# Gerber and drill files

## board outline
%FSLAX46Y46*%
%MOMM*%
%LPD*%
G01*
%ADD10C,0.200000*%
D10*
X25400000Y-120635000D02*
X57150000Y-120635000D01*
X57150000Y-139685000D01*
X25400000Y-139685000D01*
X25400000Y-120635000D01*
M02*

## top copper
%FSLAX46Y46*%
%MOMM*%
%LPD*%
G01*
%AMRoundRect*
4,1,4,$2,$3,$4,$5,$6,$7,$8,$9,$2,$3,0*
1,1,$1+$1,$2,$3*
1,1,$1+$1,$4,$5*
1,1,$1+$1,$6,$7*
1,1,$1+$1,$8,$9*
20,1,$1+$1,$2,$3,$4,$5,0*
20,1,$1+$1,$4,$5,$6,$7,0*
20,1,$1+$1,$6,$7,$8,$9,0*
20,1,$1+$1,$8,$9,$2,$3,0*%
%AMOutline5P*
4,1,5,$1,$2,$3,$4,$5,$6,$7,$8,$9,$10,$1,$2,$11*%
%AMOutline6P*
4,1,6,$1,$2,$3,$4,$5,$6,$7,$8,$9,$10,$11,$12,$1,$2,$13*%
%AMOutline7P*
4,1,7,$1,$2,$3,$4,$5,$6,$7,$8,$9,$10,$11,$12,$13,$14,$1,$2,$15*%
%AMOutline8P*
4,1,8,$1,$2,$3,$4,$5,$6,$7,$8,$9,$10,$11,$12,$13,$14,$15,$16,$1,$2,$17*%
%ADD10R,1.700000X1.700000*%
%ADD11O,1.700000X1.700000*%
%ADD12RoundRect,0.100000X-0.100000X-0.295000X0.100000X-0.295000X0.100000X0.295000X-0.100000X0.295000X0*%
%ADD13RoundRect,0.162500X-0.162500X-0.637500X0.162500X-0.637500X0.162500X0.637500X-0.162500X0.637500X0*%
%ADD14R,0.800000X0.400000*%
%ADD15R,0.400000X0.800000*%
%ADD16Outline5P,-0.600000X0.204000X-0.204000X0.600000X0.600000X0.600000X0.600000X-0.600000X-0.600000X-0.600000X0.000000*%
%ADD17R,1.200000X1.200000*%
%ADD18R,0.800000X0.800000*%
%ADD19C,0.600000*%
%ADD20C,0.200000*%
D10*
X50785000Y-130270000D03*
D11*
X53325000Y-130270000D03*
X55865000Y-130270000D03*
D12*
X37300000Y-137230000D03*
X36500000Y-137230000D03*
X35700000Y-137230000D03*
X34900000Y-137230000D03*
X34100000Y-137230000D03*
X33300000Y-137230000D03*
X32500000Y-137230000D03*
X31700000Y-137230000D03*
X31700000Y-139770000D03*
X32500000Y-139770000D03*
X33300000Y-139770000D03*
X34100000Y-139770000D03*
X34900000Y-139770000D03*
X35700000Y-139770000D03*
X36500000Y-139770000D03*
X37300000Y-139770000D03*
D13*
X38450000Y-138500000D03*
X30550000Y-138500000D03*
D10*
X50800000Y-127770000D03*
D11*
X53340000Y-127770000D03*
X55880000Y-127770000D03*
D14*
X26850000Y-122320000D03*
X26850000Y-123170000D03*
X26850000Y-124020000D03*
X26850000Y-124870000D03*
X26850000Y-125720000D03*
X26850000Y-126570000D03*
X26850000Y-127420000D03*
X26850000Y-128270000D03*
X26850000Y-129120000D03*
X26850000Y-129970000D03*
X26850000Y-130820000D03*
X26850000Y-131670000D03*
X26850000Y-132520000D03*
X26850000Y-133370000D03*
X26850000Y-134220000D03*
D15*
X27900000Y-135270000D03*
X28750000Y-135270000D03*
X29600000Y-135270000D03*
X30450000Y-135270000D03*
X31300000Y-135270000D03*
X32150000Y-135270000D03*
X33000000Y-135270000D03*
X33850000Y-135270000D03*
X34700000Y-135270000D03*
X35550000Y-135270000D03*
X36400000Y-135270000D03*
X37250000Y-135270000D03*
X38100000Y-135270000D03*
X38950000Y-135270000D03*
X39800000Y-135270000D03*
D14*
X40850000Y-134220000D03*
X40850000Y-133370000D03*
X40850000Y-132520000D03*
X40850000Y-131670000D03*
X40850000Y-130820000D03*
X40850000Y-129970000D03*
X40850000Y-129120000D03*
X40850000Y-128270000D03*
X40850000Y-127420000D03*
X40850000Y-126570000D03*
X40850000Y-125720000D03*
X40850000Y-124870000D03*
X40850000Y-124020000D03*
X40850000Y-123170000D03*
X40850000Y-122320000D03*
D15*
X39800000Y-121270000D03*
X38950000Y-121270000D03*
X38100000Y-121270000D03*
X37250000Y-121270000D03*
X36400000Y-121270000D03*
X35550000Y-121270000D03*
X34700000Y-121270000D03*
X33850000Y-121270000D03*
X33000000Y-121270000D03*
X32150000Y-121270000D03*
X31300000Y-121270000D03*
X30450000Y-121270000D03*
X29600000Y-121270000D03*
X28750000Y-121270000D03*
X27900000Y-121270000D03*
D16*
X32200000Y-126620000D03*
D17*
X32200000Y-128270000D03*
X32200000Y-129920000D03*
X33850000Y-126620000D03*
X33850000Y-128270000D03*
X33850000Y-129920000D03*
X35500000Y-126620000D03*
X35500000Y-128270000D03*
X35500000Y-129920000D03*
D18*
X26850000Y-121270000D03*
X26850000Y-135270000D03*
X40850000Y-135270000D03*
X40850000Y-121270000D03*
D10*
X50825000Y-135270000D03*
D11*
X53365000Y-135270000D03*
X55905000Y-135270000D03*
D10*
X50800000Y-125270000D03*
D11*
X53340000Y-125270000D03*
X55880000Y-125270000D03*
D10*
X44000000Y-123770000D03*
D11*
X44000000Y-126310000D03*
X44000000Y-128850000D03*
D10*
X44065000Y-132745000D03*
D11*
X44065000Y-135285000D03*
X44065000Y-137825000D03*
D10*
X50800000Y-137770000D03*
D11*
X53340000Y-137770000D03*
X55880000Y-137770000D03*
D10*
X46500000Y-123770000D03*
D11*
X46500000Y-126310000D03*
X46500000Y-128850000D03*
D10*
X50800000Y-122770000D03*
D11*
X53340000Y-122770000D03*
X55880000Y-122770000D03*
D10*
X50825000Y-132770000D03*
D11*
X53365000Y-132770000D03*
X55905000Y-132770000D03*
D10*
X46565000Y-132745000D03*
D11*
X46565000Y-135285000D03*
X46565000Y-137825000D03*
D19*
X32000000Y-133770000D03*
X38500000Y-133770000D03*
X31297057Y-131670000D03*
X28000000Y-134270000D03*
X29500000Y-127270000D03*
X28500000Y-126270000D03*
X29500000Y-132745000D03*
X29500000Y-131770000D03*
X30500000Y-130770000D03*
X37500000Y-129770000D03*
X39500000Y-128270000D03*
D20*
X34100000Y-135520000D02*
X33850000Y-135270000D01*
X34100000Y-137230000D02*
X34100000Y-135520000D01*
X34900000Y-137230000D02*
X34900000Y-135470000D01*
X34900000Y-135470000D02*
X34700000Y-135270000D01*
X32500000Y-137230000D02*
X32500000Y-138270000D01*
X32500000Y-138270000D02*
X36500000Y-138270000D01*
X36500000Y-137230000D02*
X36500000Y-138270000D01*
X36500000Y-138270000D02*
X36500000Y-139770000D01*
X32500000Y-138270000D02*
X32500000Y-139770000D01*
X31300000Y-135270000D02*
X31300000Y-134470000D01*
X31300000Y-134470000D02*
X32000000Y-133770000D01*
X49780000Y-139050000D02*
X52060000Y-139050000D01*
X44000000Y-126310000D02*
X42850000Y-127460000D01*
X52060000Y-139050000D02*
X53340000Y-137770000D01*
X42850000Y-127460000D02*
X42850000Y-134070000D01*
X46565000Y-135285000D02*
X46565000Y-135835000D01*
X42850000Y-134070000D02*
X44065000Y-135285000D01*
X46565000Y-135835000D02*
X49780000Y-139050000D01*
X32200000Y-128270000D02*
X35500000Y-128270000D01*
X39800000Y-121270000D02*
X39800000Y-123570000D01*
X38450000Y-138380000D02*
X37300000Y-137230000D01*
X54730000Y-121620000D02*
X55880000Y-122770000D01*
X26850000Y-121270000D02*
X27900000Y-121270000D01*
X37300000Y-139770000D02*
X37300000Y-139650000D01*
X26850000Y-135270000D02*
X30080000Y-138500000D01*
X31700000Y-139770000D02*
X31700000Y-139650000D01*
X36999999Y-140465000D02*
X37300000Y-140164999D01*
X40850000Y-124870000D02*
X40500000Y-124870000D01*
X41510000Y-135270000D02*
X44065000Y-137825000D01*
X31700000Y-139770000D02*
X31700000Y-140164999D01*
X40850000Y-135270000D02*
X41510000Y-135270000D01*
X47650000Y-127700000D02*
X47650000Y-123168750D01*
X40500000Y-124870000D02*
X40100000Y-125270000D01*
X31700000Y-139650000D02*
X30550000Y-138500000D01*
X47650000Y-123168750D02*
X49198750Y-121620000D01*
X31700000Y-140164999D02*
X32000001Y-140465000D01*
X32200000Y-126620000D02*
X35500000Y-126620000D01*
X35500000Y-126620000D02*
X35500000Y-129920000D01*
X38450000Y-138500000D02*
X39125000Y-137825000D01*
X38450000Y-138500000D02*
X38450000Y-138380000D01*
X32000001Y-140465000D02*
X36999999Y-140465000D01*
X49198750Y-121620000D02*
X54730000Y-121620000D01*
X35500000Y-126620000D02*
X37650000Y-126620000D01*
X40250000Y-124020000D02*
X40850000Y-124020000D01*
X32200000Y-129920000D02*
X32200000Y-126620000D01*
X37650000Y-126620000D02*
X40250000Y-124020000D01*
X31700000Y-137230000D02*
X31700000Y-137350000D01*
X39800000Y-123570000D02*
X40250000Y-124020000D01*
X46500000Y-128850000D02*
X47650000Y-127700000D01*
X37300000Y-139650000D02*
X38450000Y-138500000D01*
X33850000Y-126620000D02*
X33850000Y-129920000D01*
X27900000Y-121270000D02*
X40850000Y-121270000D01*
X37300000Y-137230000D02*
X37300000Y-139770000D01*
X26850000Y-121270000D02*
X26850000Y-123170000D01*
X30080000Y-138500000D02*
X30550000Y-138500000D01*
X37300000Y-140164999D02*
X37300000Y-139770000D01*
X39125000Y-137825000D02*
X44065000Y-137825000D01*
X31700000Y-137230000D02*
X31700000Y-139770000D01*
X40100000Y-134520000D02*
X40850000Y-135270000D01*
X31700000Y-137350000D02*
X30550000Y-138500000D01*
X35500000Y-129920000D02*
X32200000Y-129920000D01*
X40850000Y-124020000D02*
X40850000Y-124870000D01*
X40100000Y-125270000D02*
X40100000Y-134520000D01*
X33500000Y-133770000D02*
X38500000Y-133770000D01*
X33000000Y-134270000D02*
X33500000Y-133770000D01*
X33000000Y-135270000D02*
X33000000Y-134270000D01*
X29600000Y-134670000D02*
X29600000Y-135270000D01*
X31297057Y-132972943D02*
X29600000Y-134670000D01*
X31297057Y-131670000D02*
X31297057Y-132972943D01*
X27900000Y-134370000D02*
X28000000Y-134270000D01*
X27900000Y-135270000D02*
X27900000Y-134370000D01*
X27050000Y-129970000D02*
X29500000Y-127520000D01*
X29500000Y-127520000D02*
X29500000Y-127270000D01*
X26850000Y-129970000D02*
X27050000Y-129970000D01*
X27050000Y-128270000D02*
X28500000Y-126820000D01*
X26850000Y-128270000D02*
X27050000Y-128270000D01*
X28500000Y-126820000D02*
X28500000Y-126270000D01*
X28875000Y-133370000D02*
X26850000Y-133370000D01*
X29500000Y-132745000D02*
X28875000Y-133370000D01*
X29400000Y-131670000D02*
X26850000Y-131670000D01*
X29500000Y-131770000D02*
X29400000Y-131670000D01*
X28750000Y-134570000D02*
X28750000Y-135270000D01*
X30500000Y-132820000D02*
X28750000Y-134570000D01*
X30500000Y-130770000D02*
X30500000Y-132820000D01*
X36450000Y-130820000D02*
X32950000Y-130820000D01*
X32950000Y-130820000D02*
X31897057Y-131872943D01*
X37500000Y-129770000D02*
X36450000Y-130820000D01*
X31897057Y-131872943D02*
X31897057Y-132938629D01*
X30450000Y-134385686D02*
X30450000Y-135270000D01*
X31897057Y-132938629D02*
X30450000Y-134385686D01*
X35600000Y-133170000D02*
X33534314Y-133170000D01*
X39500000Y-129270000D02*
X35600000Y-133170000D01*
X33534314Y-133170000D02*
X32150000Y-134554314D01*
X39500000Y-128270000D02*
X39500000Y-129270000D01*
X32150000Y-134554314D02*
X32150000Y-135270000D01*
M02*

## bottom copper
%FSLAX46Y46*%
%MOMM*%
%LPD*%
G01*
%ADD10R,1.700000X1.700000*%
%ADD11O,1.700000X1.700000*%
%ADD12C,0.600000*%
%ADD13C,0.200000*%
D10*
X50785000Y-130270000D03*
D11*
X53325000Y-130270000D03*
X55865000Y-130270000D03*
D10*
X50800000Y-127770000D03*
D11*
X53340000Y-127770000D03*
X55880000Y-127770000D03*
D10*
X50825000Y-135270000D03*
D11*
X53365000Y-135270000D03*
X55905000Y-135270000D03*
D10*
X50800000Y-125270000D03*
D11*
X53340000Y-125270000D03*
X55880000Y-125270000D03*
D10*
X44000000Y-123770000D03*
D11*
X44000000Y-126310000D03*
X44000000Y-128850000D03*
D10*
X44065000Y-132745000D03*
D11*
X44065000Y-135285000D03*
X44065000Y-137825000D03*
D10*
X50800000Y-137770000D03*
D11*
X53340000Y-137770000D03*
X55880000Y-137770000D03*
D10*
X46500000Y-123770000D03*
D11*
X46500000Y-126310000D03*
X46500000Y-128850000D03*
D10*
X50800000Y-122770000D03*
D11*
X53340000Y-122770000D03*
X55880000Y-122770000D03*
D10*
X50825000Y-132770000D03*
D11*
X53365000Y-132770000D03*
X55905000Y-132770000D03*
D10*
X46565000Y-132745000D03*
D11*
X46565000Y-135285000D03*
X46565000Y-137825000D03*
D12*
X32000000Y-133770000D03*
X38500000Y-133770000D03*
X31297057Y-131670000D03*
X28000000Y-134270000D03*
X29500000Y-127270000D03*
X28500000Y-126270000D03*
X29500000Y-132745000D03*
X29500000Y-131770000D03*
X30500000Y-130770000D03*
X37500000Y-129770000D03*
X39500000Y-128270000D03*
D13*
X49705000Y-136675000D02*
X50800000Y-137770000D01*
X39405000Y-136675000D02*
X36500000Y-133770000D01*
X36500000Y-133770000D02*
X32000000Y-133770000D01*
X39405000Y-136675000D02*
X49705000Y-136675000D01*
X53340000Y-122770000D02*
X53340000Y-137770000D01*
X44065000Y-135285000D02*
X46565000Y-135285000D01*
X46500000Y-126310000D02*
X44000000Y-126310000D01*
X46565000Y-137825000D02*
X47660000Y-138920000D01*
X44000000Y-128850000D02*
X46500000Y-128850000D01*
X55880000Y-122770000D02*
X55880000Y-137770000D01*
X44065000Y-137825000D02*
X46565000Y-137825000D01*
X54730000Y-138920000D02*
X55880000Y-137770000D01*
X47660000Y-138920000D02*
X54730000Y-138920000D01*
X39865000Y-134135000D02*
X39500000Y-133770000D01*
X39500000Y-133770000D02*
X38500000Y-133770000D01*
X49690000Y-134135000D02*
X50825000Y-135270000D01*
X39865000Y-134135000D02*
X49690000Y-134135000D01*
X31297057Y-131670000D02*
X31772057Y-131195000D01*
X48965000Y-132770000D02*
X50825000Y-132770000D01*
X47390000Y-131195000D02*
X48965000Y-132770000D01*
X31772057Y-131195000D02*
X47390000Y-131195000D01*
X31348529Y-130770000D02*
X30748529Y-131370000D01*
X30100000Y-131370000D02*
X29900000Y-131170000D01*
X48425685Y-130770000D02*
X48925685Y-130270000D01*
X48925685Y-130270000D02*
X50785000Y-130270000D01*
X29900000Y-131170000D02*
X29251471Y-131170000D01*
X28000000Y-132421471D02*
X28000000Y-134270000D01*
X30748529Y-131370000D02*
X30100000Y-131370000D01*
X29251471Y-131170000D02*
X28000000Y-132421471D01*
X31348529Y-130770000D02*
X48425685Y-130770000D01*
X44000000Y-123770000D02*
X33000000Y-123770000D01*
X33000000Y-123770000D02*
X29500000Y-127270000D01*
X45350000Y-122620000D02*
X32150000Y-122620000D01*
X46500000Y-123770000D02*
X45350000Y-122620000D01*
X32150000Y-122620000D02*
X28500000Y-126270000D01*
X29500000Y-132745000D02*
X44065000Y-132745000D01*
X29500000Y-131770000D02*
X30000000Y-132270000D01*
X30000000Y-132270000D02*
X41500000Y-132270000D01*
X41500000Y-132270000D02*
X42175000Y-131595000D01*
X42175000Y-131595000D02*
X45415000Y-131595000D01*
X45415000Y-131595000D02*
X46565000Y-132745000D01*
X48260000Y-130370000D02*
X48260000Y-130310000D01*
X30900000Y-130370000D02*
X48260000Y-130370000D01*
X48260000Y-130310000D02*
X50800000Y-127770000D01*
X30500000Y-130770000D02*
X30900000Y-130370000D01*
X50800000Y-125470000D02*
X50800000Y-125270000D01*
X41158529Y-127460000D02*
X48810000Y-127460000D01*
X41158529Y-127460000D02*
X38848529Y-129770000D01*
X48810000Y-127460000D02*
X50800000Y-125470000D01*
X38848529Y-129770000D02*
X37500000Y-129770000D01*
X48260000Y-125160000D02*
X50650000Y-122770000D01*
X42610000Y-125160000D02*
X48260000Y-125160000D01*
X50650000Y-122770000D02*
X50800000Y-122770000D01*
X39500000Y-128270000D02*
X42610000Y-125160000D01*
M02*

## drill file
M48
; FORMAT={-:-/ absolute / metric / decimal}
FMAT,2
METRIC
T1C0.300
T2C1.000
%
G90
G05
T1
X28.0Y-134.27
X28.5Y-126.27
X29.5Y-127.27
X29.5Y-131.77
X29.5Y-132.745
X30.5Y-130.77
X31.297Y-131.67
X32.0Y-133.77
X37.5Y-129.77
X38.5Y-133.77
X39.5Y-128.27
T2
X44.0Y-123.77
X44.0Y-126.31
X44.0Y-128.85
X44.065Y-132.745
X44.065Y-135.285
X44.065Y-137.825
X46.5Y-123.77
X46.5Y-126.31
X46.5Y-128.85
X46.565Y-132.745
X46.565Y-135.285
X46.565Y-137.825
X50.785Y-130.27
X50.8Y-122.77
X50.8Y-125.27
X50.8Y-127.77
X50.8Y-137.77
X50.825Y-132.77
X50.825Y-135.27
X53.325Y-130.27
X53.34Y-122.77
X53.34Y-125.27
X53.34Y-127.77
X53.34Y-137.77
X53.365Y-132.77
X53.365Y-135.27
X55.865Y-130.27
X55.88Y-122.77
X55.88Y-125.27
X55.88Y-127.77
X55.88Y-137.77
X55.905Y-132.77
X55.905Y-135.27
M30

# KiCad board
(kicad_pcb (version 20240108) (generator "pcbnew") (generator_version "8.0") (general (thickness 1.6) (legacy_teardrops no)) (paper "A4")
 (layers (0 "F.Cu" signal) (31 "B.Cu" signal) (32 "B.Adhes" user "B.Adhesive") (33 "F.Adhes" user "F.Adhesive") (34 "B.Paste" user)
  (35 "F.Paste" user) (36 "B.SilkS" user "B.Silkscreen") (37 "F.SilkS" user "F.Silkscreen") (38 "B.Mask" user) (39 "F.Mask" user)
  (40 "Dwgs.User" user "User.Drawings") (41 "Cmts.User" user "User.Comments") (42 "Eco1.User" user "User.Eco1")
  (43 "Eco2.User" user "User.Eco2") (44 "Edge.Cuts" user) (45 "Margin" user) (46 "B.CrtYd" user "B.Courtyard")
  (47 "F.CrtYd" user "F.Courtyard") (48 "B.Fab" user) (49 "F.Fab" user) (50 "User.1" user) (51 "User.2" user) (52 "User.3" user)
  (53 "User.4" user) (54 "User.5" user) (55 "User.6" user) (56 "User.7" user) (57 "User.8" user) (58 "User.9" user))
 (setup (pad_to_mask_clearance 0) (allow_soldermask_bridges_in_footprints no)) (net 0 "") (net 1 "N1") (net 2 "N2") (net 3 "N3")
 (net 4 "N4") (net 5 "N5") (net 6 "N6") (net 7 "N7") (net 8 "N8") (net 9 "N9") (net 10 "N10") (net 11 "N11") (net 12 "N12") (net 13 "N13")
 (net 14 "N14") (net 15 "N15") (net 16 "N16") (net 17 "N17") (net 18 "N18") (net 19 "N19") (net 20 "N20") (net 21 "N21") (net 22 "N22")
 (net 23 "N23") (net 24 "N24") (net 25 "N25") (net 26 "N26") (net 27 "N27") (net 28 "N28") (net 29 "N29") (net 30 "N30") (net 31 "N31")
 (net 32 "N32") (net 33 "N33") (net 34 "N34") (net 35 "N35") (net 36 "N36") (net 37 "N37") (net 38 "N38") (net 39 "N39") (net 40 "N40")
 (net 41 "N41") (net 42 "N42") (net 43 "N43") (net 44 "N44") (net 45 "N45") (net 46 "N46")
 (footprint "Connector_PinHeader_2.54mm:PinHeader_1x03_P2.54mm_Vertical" (layer "F.Cu") (at 50.785 130.27 90)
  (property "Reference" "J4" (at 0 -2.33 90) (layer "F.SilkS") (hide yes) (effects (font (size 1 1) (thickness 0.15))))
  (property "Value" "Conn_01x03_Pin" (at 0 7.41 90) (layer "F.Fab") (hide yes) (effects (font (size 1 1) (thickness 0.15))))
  (pad "1" thru_hole rect (at 0 0 90) (size 1.7 1.7) (drill 1) (layers "*.Cu" "*.Mask") (remove_unused_layers no) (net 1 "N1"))
  (pad "2" thru_hole oval (at 0 2.54 90) (size 1.7 1.7) (drill 1) (layers "*.Cu" "*.Mask") (remove_unused_layers no) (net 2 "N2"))
  (pad "3" thru_hole oval (at 0 5.08 90) (size 1.7 1.7) (drill 1) (layers "*.Cu" "*.Mask") (remove_unused_layers no) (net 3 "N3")))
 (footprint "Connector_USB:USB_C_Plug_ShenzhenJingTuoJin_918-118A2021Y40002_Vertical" (layer "F.Cu") (at 34.5 138.5 -90)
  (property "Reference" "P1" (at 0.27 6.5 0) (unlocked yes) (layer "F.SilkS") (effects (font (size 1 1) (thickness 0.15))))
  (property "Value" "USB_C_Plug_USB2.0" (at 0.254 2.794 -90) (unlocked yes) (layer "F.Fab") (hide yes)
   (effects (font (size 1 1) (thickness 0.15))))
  (pad "A1" smd roundrect (at -1.27 -2.8) (size 0.4 0.79) (layers "F.Cu" "F.Paste" "F.Mask") (roundrect_rratio 0.25) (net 3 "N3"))
  (pad "A4" smd roundrect (at -1.27 -2) (size 0.4 0.79) (layers "F.Cu" "F.Paste" "F.Mask") (roundrect_rratio 0.25) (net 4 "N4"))
  (pad "A5" smd roundrect (at -1.27 -1.2) (size 0.4 0.79) (layers "F.Cu" "F.Paste" "F.Mask") (roundrect_rratio 0.25) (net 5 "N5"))
  (pad "A6" smd roundrect (at -1.27 -0.4) (size 0.4 0.79) (layers "F.Cu" "F.Paste" "F.Mask") (roundrect_rratio 0.25) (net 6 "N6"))
  (pad "A7" smd roundrect (at -1.27 0.4) (size 0.4 0.79) (layers "F.Cu" "F.Paste" "F.Mask") (roundrect_rratio 0.25) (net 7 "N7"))
  (pad "A8" smd roundrect (at -1.27 1.2) (size 0.4 0.79) (layers "F.Cu" "F.Paste" "F.Mask") (roundrect_rratio 0.25))
  (pad "A9" smd roundrect (at -1.27 2) (size 0.4 0.79) (layers "F.Cu" "F.Paste" "F.Mask") (roundrect_rratio 0.25) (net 4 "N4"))
  (pad "A12" smd roundrect (at -1.27 2.8) (size 0.4 0.79) (layers "F.Cu" "F.Paste" "F.Mask") (roundrect_rratio 0.25) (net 3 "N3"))
  (pad "B1" smd roundrect (at 1.27 2.8) (size 0.4 0.79) (layers "F.Cu" "F.Paste" "F.Mask") (roundrect_rratio 0.25) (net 3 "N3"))
  (pad "B4" smd roundrect (at 1.27 2) (size 0.4 0.79) (layers "F.Cu" "F.Paste" "F.Mask") (roundrect_rratio 0.25) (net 4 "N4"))
  (pad "B5" smd roundrect (at 1.27 1.2) (size 0.4 0.79) (layers "F.Cu" "F.Paste" "F.Mask") (roundrect_rratio 0.25) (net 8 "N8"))
  (pad "B6" smd roundrect (at 1.27 0.4) (size 0.4 0.79) (layers "F.Cu" "F.Paste" "F.Mask") (roundrect_rratio 0.25))
  (pad "B7" smd roundrect (at 1.27 -0.4) (size 0.4 0.79) (layers "F.Cu" "F.Paste" "F.Mask") (roundrect_rratio 0.25))
  (pad "B8" smd roundrect (at 1.27 -1.2) (size 0.4 0.79) (layers "F.Cu" "F.Paste" "F.Mask") (roundrect_rratio 0.25))
  (pad "B9" smd roundrect (at 1.27 -2) (size 0.4 0.79) (layers "F.Cu" "F.Paste" "F.Mask") (roundrect_rratio 0.25) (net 4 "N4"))
  (pad "B12" smd roundrect (at 1.27 -2.8) (size 0.4 0.79) (layers "F.Cu" "F.Paste" "F.Mask") (roundrect_rratio 0.25) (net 3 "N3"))
  (pad "S1" smd roundrect (at 0 -3.95) (size 0.65 1.6) (layers "F.Cu" "F.Paste" "F.Mask") (roundrect_rratio 0.25) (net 3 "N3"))
  (pad "S1" smd roundrect (at 0 3.95) (size 0.65 1.6) (layers "F.Cu" "F.Paste" "F.Mask") (roundrect_rratio 0.25) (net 3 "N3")))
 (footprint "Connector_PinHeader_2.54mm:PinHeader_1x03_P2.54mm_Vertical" (layer "F.Cu") (at 50.8 127.77 90)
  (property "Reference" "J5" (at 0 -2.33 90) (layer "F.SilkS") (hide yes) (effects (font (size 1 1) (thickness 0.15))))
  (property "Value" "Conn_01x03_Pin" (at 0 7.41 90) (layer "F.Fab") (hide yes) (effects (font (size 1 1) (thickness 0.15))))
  (pad "1" thru_hole rect (at 0 0 90) (size 1.7 1.7) (drill 1) (layers "*.Cu" "*.Mask") (remove_unused_layers no) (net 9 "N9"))
  (pad "2" thru_hole oval (at 0 2.54 90) (size 1.7 1.7) (drill 1) (layers "*.Cu" "*.Mask") (remove_unused_layers no) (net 2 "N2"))
  (pad "3" thru_hole oval (at 0 5.08 90) (size 1.7 1.7) (drill 1) (layers "*.Cu" "*.Mask") (remove_unused_layers no) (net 3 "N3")))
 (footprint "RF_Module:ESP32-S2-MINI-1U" (layer "F.Cu") (at 33.85 128.27)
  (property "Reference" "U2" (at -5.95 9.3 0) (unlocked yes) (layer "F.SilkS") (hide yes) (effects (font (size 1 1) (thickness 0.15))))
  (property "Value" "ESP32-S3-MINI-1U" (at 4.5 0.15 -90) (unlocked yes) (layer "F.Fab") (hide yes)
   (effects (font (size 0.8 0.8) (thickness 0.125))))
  (pad "1" smd rect (at -7 -5.95) (size 0.8 0.4) (layers "F.Cu" "F.Paste" "F.Mask") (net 3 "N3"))
  (pad "2" smd rect (at -7 -5.1) (size 0.8 0.4) (layers "F.Cu" "F.Paste" "F.Mask") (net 3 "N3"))
  (pad "3" smd rect (at -7 -4.25) (size 0.8 0.4) (layers "F.Cu" "F.Paste" "F.Mask") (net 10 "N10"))
  (pad "4" smd rect (at -7 -3.4) (size 0.8 0.4) (layers "F.Cu" "F.Paste" "F.Mask") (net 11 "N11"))
  (pad "5" smd rect (at -7 -2.55) (size 0.8 0.4) (layers "F.Cu" "F.Paste" "F.Mask") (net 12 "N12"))
  (pad "6" smd rect (at -7 -1.7) (size 0.8 0.4) (layers "F.Cu" "F.Paste" "F.Mask") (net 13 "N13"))
  (pad "7" smd rect (at -7 -0.85) (size 0.8 0.4) (layers "F.Cu" "F.Paste" "F.Mask") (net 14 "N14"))
  (pad "8" smd rect (at -7 0) (size 0.8 0.4) (layers "F.Cu" "F.Paste" "F.Mask") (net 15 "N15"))
  (pad "9" smd rect (at -7 0.85) (size 0.8 0.4) (layers "F.Cu" "F.Paste" "F.Mask") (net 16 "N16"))
  (pad "10" smd rect (at -7 1.7) (size 0.8 0.4) (layers "F.Cu" "F.Paste" "F.Mask") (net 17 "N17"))
  (pad "11" smd rect (at -7 2.55) (size 0.8 0.4) (layers "F.Cu" "F.Paste" "F.Mask") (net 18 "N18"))
  (pad "12" smd rect (at -7 3.4) (size 0.8 0.4) (layers "F.Cu" "F.Paste" "F.Mask") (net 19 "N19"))
  (pad "13" smd rect (at -7 4.25) (size 0.8 0.4) (layers "F.Cu" "F.Paste" "F.Mask") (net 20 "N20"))
  (pad "14" smd rect (at -7 5.1) (size 0.8 0.4) (layers "F.Cu" "F.Paste" "F.Mask") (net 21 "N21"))
  (pad "15" smd rect (at -7 5.95) (size 0.8 0.4) (layers "F.Cu" "F.Paste" "F.Mask") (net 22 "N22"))
  (pad "16" smd rect (at -5.95 7 90) (size 0.8 0.4) (layers "F.Cu" "F.Paste" "F.Mask") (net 1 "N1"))
  (pad "17" smd rect (at -5.1 7 90) (size 0.8 0.4) (layers "F.Cu" "F.Paste" "F.Mask") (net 9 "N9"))
  (pad "18" smd rect (at -4.25 7 90) (size 0.8 0.4) (layers "F.Cu" "F.Paste" "F.Mask") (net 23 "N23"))
  (pad "19" smd rect (at -3.4 7 90) (size 0.8 0.4) (layers "F.Cu" "F.Paste" "F.Mask") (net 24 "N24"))
  (pad "20" smd rect (at -2.55 7 90) (size 0.8 0.4) (layers "F.Cu" "F.Paste" "F.Mask") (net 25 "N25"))
  (pad "21" smd rect (at -1.7 7 90) (size 0.8 0.4) (layers "F.Cu" "F.Paste" "F.Mask") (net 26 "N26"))
  (pad "22" smd rect (at -0.85 7 90) (size 0.8 0.4) (layers "F.Cu" "F.Paste" "F.Mask") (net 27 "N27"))
  (pad "23" smd rect (at 0 7 90) (size 0.8 0.4) (layers "F.Cu" "F.Paste" "F.Mask") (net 7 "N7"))
  (pad "24" smd rect (at 0.85 7 90) (size 0.8 0.4) (layers "F.Cu" "F.Paste" "F.Mask") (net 6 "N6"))
  (pad "25" smd rect (at 1.7 7 90) (size 0.8 0.4) (layers "F.Cu" "F.Paste" "F.Mask") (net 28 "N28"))
  (pad "26" smd rect (at 2.55 7 90) (size 0.8 0.4) (layers "F.Cu" "F.Paste" "F.Mask") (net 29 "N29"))
  (pad "27" smd rect (at 3.4 7 90) (size 0.8 0.4) (layers "F.Cu" "F.Paste" "F.Mask") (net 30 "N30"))
  (pad "28" smd rect (at 4.25 7 90) (size 0.8 0.4) (layers "F.Cu" "F.Paste" "F.Mask") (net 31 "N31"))
  (pad "29" smd rect (at 5.1 7 90) (size 0.8 0.4) (layers "F.Cu" "F.Paste" "F.Mask") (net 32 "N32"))
  (pad "30" smd rect (at 5.95 7 90) (size 0.8 0.4) (layers "F.Cu" "F.Paste" "F.Mask") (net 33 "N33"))
  (pad "31" smd rect (at 7 5.95) (size 0.8 0.4) (layers "F.Cu" "F.Paste" "F.Mask") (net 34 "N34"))
  (pad "32" smd rect (at 7 5.1) (size 0.8 0.4) (layers "F.Cu" "F.Paste" "F.Mask") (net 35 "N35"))
  (pad "33" smd rect (at 7 4.25) (size 0.8 0.4) (layers "F.Cu" "F.Paste" "F.Mask") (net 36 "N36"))
  (pad "34" smd rect (at 7 3.4) (size 0.8 0.4) (layers "F.Cu" "F.Paste" "F.Mask") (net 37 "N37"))
  (pad "35" smd rect (at 7 2.55) (size 0.8 0.4) (layers "F.Cu" "F.Paste" "F.Mask") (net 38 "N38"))
  (pad "36" smd rect (at 7 1.7) (size 0.8 0.4) (layers "F.Cu" "F.Paste" "F.Mask") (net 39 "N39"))
  (pad "37" smd rect (at 7 0.85) (size 0.8 0.4) (layers "F.Cu" "F.Paste" "F.Mask") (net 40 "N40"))
  (pad "38" smd rect (at 7 0) (size 0.8 0.4) (layers "F.Cu" "F.Paste" "F.Mask") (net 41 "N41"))
  (pad "39" smd rect (at 7 -0.85) (size 0.8 0.4) (layers "F.Cu" "F.Paste" "F.Mask") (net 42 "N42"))
  (pad "40" smd rect (at 7 -1.7) (size 0.8 0.4) (layers "F.Cu" "F.Paste" "F.Mask") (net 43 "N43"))
  (pad "41" smd rect (at 7 -2.55) (size 0.8 0.4) (layers "F.Cu" "F.Paste" "F.Mask") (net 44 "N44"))
  (pad "42" smd rect (at 7 -3.4) (size 0.8 0.4) (layers "F.Cu" "F.Paste" "F.Mask") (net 3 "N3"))
  (pad "43" smd rect (at 7 -4.25) (size 0.8 0.4) (layers "F.Cu" "F.Paste" "F.Mask") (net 3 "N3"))
  (pad "44" smd rect (at 7 -5.1) (size 0.8 0.4) (layers "F.Cu" "F.Paste" "F.Mask") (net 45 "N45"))
  (pad "45" smd rect (at 7 -5.95) (size 0.8 0.4) (layers "F.Cu" "F.Paste" "F.Mask") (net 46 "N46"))
  (pad "46" smd rect (at 5.95 -7 90) (size 0.8 0.4) (layers "F.Cu" "F.Paste" "F.Mask") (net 3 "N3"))
  (pad "47" smd rect (at 5.1 -7 90) (size 0.8 0.4) (layers "F.Cu" "F.Paste" "F.Mask") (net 3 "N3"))
  (pad "48" smd rect (at 4.25 -7 90) (size 0.8 0.4) (layers "F.Cu" "F.Paste" "F.Mask") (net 3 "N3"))
  (pad "49" smd rect (at 3.4 -7 90) (size 0.8 0.4) (layers "F.Cu" "F.Paste" "F.Mask") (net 3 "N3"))
  (pad "50" smd rect (at 2.55 -7 90) (size 0.8 0.4) (layers "F.Cu" "F.Paste" "F.Mask") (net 3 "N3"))
  (pad "51" smd rect (at 1.7 -7 90) (size 0.8 0.4) (layers "F.Cu" "F.Paste" "F.Mask") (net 3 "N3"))
  (pad "52" smd rect (at 0.85 -7 90) (size 0.8 0.4) (layers "F.Cu" "F.Paste" "F.Mask") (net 3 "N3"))
  (pad "53" smd rect (at 0 -7 90) (size 0.8 0.4) (layers "F.Cu" "F.Paste" "F.Mask") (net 3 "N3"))
  (pad "54" smd rect (at -0.85 -7 90) (size 0.8 0.4) (layers "F.Cu" "F.Paste" "F.Mask") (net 3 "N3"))
  (pad "55" smd rect (at -1.7 -7 90) (size 0.8 0.4) (layers "F.Cu" "F.Paste" "F.Mask") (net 3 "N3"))
  (pad "56" smd rect (at -2.55 -7 90) (size 0.8 0.4) (layers "F.Cu" "F.Paste" "F.Mask") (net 3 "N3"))
  (pad "57" smd rect (at -3.4 -7 90) (size 0.8 0.4) (layers "F.Cu" "F.Paste" "F.Mask") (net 3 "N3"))
  (pad "58" smd rect (at -4.25 -7 90) (size 0.8 0.4) (layers "F.Cu" "F.Paste" "F.Mask") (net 3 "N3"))
  (pad "59" smd rect (at -5.1 -7 90) (size 0.8 0.4) (layers "F.Cu" "F.Paste" "F.Mask") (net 3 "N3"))
  (pad "60" smd rect (at -5.95 -7 90) (size 0.8 0.4) (layers "F.Cu" "F.Paste" "F.Mask") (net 3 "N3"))
  (pad "61" smd roundrect (at -1.65 -1.65) (size 1.2 1.2) (layers "F.Cu" "F.Paste" "F.Mask") (roundrect_rratio 0) (chamfer_ratio 0.33)
   (chamfer top_left) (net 3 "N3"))
  (pad "61" smd rect (at -1.65 0) (size 1.2 1.2) (layers "F.Cu" "F.Paste" "F.Mask") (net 3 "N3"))
  (pad "61" smd rect (at -1.65 1.65) (size 1.2 1.2) (layers "F.Cu" "F.Paste" "F.Mask") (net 3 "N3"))
  (pad "61" smd rect (at 0 -1.65) (size 1.2 1.2) (layers "F.Cu" "F.Paste" "F.Mask") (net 3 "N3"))
  (pad "61" smd rect (at 0 0) (size 1.2 1.2) (layers "F.Cu" "F.Paste" "F.Mask") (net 3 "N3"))
  (pad "61" smd rect (at 0 1.65) (size 1.2 1.2) (layers "F.Cu" "F.Paste" "F.Mask") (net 3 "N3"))
  (pad "61" smd rect (at 1.65 -1.65) (size 1.2 1.2) (layers "F.Cu" "F.Paste" "F.Mask") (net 3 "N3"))
  (pad "61" smd rect (at 1.65 0) (size 1.2 1.2) (layers "F.Cu" "F.Paste" "F.Mask") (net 3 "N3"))
  (pad "61" smd rect (at 1.65 1.65) (size 1.2 1.2) (layers "F.Cu" "F.Paste" "F.Mask") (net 3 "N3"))
  (pad "62" smd rect (at -7 -7) (size 0.8 0.8) (layers "F.Cu" "F.Paste" "F.Mask") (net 3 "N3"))
  (pad "63" smd rect (at -7 7) (size 0.8 0.8) (layers "F.Cu" "F.Paste" "F.Mask") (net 3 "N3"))
  (pad "64" smd rect (at 7 7) (size 0.8 0.8) (layers "F.Cu" "F.Paste" "F.Mask") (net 3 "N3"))
  (pad "65" smd rect (at 7 -7) (size 0.8 0.8) (layers "F.Cu" "F.Paste" "F.Mask") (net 3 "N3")))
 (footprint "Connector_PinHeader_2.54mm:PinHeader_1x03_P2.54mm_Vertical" (layer "F.Cu") (at 50.825 135.27 90)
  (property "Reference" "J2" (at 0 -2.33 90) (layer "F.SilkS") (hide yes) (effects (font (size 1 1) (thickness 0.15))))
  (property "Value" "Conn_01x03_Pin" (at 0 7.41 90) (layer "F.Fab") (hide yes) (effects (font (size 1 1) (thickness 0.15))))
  (pad "1" thru_hole rect (at 0 0 90) (size 1.7 1.7) (drill 1) (layers "*.Cu" "*.Mask") (remove_unused_layers no) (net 27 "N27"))
  (pad "2" thru_hole oval (at 0 2.54 90) (size 1.7 1.7) (drill 1) (layers "*.Cu" "*.Mask") (remove_unused_layers no) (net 2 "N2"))
  (pad "3" thru_hole oval (at 0 5.08 90) (size 1.7 1.7) (drill 1) (layers "*.Cu" "*.Mask") (remove_unused_layers no) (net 3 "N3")))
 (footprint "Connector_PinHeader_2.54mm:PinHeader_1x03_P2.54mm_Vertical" (layer "F.Cu") (at 50.8 125.27 90)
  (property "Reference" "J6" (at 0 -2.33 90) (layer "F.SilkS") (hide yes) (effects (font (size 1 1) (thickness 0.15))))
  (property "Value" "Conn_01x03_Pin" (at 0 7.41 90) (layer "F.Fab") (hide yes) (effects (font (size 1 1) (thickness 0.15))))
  (pad "1" thru_hole rect (at 0 0 90) (size 1.7 1.7) (drill 1) (layers "*.Cu" "*.Mask") (remove_unused_layers no) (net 24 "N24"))
  (pad "2" thru_hole oval (at 0 2.54 90) (size 1.7 1.7) (drill 1) (layers "*.Cu" "*.Mask") (remove_unused_layers no) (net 2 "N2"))
  (pad "3" thru_hole oval (at 0 5.08 90) (size 1.7 1.7) (drill 1) (layers "*.Cu" "*.Mask") (remove_unused_layers no) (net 3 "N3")))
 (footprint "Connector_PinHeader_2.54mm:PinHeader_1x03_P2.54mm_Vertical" (layer "F.Cu") (at 44 123.77)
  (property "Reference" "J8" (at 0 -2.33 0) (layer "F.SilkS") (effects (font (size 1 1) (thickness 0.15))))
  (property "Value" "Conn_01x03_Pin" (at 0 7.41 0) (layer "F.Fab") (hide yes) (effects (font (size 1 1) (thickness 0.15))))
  (pad "1" thru_hole rect (at 0 0) (size 1.7 1.7) (drill 1) (layers "*.Cu" "*.Mask") (remove_unused_layers no) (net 17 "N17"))
  (pad "2" thru_hole oval (at 0 2.54) (size 1.7 1.7) (drill 1) (layers "*.Cu" "*.Mask") (remove_unused_layers no) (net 2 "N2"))
  (pad "3" thru_hole oval (at 0 5.08) (size 1.7 1.7) (drill 1) (layers "*.Cu" "*.Mask") (remove_unused_layers no) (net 3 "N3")))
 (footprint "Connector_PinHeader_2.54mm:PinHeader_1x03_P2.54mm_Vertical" (layer "F.Cu") (at 44.065 132.745)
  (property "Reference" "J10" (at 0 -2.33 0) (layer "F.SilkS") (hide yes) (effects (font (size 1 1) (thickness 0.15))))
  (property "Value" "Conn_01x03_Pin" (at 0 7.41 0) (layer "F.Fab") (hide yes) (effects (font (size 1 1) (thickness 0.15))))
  (pad "1" thru_hole rect (at 0 0) (size 1.7 1.7) (drill 1) (layers "*.Cu" "*.Mask") (remove_unused_layers no) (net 21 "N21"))
  (pad "2" thru_hole oval (at 0 2.54) (size 1.7 1.7) (drill 1) (layers "*.Cu" "*.Mask") (remove_unused_layers no) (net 2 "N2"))
  (pad "3" thru_hole oval (at 0 5.08) (size 1.7 1.7) (drill 1) (layers "*.Cu" "*.Mask") (remove_unused_layers no) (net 3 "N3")))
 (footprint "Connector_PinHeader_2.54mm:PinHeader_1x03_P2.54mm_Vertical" (layer "F.Cu") (at 50.8 137.77 90)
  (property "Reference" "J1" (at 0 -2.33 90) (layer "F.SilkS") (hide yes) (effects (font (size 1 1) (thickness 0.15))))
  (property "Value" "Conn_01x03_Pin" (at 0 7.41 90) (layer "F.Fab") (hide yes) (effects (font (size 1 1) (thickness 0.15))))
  (pad "1" thru_hole rect (at 0 0 90) (size 1.7 1.7) (drill 1) (layers "*.Cu" "*.Mask") (remove_unused_layers no) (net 25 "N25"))
  (pad "2" thru_hole oval (at 0 2.54 90) (size 1.7 1.7) (drill 1) (layers "*.Cu" "*.Mask") (remove_unused_layers no) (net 2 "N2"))
  (pad "3" thru_hole oval (at 0 5.08 90) (size 1.7 1.7) (drill 1) (layers "*.Cu" "*.Mask") (remove_unused_layers no) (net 3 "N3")))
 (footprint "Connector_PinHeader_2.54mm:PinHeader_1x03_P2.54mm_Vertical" (layer "F.Cu") (at 46.5 123.77)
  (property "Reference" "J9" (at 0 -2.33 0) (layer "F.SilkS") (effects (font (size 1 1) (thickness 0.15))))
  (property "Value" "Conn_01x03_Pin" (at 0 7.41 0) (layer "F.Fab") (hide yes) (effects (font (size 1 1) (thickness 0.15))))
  (pad "1" thru_hole rect (at 0 0) (size 1.7 1.7) (drill 1) (layers "*.Cu" "*.Mask") (remove_unused_layers no) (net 15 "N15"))
  (pad "2" thru_hole oval (at 0 2.54) (size 1.7 1.7) (drill 1) (layers "*.Cu" "*.Mask") (remove_unused_layers no) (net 2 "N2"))
  (pad "3" thru_hole oval (at 0 5.08) (size 1.7 1.7) (drill 1) (layers "*.Cu" "*.Mask") (remove_unused_layers no) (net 3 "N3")))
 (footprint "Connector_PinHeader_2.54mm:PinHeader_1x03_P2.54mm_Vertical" (layer "F.Cu") (at 50.8 122.77 90)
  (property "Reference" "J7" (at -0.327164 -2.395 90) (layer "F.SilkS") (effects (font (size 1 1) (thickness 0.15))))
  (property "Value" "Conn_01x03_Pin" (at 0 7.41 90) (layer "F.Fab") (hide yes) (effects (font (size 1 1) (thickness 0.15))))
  (pad "1" thru_hole rect (at 0 0 90) (size 1.7 1.7) (drill 1) (layers "*.Cu" "*.Mask") (remove_unused_layers no) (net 26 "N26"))
  (pad "2" thru_hole oval (at 0 2.54 90) (size 1.7 1.7) (drill 1) (layers "*.Cu" "*.Mask") (remove_unused_layers no) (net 2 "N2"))
  (pad "3" thru_hole oval (at 0 5.08 90) (size 1.7 1.7) (drill 1) (layers "*.Cu" "*.Mask") (remove_unused_layers no) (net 3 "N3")))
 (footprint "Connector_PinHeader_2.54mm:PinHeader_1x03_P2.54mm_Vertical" (layer "F.Cu") (at 50.825 132.77 90)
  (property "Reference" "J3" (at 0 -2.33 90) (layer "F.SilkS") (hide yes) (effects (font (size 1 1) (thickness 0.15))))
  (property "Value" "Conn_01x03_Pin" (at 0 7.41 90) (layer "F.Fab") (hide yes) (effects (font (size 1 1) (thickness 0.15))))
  (pad "1" thru_hole rect (at 0 0 90) (size 1.7 1.7) (drill 1) (layers "*.Cu" "*.Mask") (remove_unused_layers no) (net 23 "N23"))
  (pad "2" thru_hole oval (at 0 2.54 90) (size 1.7 1.7) (drill 1) (layers "*.Cu" "*.Mask") (remove_unused_layers no) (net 2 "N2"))
  (pad "3" thru_hole oval (at 0 5.08 90) (size 1.7 1.7) (drill 1) (layers "*.Cu" "*.Mask") (remove_unused_layers no) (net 3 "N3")))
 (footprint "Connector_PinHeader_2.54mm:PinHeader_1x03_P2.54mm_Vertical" (layer "F.Cu") (at 46.565 132.745)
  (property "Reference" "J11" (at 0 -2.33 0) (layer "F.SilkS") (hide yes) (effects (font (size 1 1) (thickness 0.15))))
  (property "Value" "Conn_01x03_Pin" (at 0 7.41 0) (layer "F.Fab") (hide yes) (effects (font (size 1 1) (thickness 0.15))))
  (pad "1" thru_hole rect (at 0 0) (size 1.7 1.7) (drill 1) (layers "*.Cu" "*.Mask") (remove_unused_layers no) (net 19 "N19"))
  (pad "2" thru_hole oval (at 0 2.54) (size 1.7 1.7) (drill 1) (layers "*.Cu" "*.Mask") (remove_unused_layers no) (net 2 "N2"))
  (pad "3" thru_hole oval (at 0 5.08) (size 1.7 1.7) (drill 1) (layers "*.Cu" "*.Mask") (remove_unused_layers no) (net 3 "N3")))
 (gr_rect (start 25.4 120.635) (end 57.15 139.685) (stroke (width 0.2) (type default)) (fill none) (layer "Edge.Cuts"))
 (segment (start 34.1 135.52) (end 33.85 135.27) (width 0.2) (layer "F.Cu") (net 7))
 (segment (start 34.1 137.23) (end 34.1 135.52) (width 0.2) (layer "F.Cu") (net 7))
 (segment (start 34.9 137.23) (end 34.9 135.47) (width 0.2) (layer "F.Cu") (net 6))
 (segment (start 34.9 135.47) (end 34.7 135.27) (width 0.2) (layer "F.Cu") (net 6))
 (segment (start 32.5 137.23) (end 32.5 138.27) (width 0.2) (layer "F.Cu") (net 4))
 (segment (start 32.5 138.27) (end 36.5 138.27) (width 0.2) (layer "F.Cu") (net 4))
 (segment (start 36.5 137.23) (end 36.5 138.27) (width 0.2) (layer "F.Cu") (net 4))
 (segment (start 36.5 138.27) (end 36.5 139.77) (width 0.2) (layer "F.Cu") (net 4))
 (segment (start 32.5 138.27) (end 32.5 139.77) (width 0.2) (layer "F.Cu") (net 4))
 (segment (start 31.3 135.27) (end 31.3 134.47) (width 0.2) (layer "F.Cu") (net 25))
 (segment (start 31.3 134.47) (end 32 133.77) (width 0.2) (layer "F.Cu") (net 25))
 (via (at 32 133.77) (size 0.6) (drill 0.3) (layers "F.Cu" "B.Cu") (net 25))
 (segment (start 49.705 136.675) (end 50.8 137.77) (width 0.2) (layer "B.Cu") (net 25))
 (segment (start 39.405 136.675) (end 36.5 133.77) (width 0.2) (layer "B.Cu") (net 25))
 (segment (start 36.5 133.77) (end 32 133.77) (width 0.2) (layer "B.Cu") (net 25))
 (segment (start 39.405 136.675) (end 49.705 136.675) (width 0.2) (layer "B.Cu") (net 25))
 (segment (start 49.78 139.05) (end 52.06 139.05) (width 0.2) (layer "F.Cu") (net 2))
 (segment (start 44 126.31) (end 42.85 127.46) (width 0.2) (layer "F.Cu") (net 2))
 (segment (start 52.06 139.05) (end 53.34 137.77) (width 0.2) (layer "F.Cu") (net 2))
 (segment (start 42.85 127.46) (end 42.85 134.07) (width 0.2) (layer "F.Cu") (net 2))
 (segment (start 46.565 135.285) (end 46.565 135.835) (width 0.2) (layer "F.Cu") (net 2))
 (segment (start 42.85 134.07) (end 44.065 135.285) (width 0.2) (layer "F.Cu") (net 2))
 (segment (start 46.565 135.835) (end 49.78 139.05) (width 0.2) (layer "F.Cu") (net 2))
 (segment (start 53.34 122.77) (end 53.34 137.77) (width 0.2) (layer "B.Cu") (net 2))
 (segment (start 44.065 135.285) (end 46.565 135.285) (width 0.2) (layer "B.Cu") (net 2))
 (segment (start 46.5 126.31) (end 44 126.31) (width 0.2) (layer "B.Cu") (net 2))
 (segment (start 32.2 128.27) (end 35.5 128.27) (width 0.2) (layer "F.Cu") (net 3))
 (segment (start 39.8 121.27) (end 39.8 123.57) (width 0.2) (layer "F.Cu") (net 3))
 (segment (start 38.45 138.38) (end 37.3 137.23) (width 0.2) (layer "F.Cu") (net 3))
 (segment (start 54.73 121.62) (end 55.88 122.77) (width 0.2) (layer "F.Cu") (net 3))
 (segment (start 26.85 121.27) (end 27.9 121.27) (width 0.2) (layer "F.Cu") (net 3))
 (segment (start 37.3 139.77) (end 37.3 139.65) (width 0.2) (layer "F.Cu") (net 3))
 (segment (start 26.85 135.27) (end 30.08 138.5) (width 0.2) (layer "F.Cu") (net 3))
 (segment (start 31.7 139.77) (end 31.7 139.65) (width 0.2) (layer "F.Cu") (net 3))
 (segment (start 36.999999 140.465) (end 37.3 140.164999) (width 0.2) (layer "F.Cu") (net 3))
 (segment (start 40.85 124.87) (end 40.5 124.87) (width 0.2) (layer "F.Cu") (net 3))
 (segment (start 41.51 135.27) (end 44.065 137.825) (width 0.2) (layer "F.Cu") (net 3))
 (segment (start 31.7 139.77) (end 31.7 140.164999) (width 0.2) (layer "F.Cu") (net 3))
 (segment (start 40.85 135.27) (end 41.51 135.27) (width 0.2) (layer "F.Cu") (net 3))
 (segment (start 47.65 127.7) (end 47.65 123.16875) (width 0.2) (layer "F.Cu") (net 3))
 (segment (start 40.5 124.87) (end 40.1 125.27) (width 0.2) (layer "F.Cu") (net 3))
 (segment (start 31.7 139.65) (end 30.55 138.5) (width 0.2) (layer "F.Cu") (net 3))
 (segment (start 47.65 123.16875) (end 49.19875 121.62) (width 0.2) (layer "F.Cu") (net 3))
 (segment (start 31.7 140.164999) (end 32.000001 140.465) (width 0.2) (layer "F.Cu") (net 3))
 (segment (start 32.2 126.62) (end 35.5 126.62) (width 0.2) (layer "F.Cu") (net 3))
 (segment (start 35.5 126.62) (end 35.5 129.92) (width 0.2) (layer "F.Cu") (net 3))
 (segment (start 38.45 138.5) (end 39.125 137.825) (width 0.2) (layer "F.Cu") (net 3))
 (segment (start 38.45 138.5) (end 38.45 138.38) (width 0.2) (layer "F.Cu") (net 3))
 (segment (start 32.000001 140.465) (end 36.999999 140.465) (width 0.2) (layer "F.Cu") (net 3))
 (segment (start 49.19875 121.62) (end 54.73 121.62) (width 0.2) (layer "F.Cu") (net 3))
 (segment (start 35.5 126.62) (end 37.65 126.62) (width 0.2) (layer "F.Cu") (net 3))
 (segment (start 40.25 124.02) (end 40.85 124.02) (width 0.2) (layer "F.Cu") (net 3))
 (segment (start 32.2 129.92) (end 32.2 126.62) (width 0.2) (layer "F.Cu") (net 3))
 (segment (start 37.65 126.62) (end 40.25 124.02) (width 0.2) (layer "F.Cu") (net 3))
 (segment (start 31.7 137.23) (end 31.7 137.35) (width 0.2) (layer "F.Cu") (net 3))
 (segment (start 39.8 123.57) (end 40.25 124.02) (width 0.2) (layer "F.Cu") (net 3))
 (segment (start 46.5 128.85) (end 47.65 127.7) (width 0.2) (layer "F.Cu") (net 3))
 (segment (start 37.3 139.65) (end 38.45 138.5) (width 0.2) (layer "F.Cu") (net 3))
 (segment (start 33.85 126.62) (end 33.85 129.92) (width 0.2) (layer "F.Cu") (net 3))
 (segment (start 27.9 121.27) (end 40.85 121.27) (width 0.2) (layer "F.Cu") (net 3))
 (segment (start 37.3 137.23) (end 37.3 139.77) (width 0.2) (layer "F.Cu") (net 3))
 (segment (start 26.85 121.27) (end 26.85 123.17) (width 0.2) (layer "F.Cu") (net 3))
 (segment (start 30.08 138.5) (end 30.55 138.5) (width 0.2) (layer "F.Cu") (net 3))
 (segment (start 37.3 140.164999) (end 37.3 139.77) (width 0.2) (layer "F.Cu") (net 3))
 (segment (start 39.125 137.825) (end 44.065 137.825) (width 0.2) (layer "F.Cu") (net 3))
 (segment (start 31.7 137.23) (end 31.7 139.77) (width 0.2) (layer "F.Cu") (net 3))
 (segment (start 40.1 134.52) (end 40.85 135.27) (width 0.2) (layer "F.Cu") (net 3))
 (segment (start 31.7 137.35) (end 30.55 138.5) (width 0.2) (layer "F.Cu") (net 3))
 (segment (start 35.5 129.92) (end 32.2 129.92) (width 0.2) (layer "F.Cu") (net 3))
 (segment (start 40.85 124.02) (end 40.85 124.87) (width 0.2) (layer "F.Cu") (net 3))
 (segment (start 40.1 125.27) (end 40.1 134.52) (width 0.2) (layer "F.Cu") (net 3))
 (segment (start 46.565 137.825) (end 47.66 138.92) (width 0.2) (layer "B.Cu") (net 3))
 (segment (start 44 128.85) (end 46.5 128.85) (width 0.2) (layer "B.Cu") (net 3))
 (segment (start 55.88 122.77) (end 55.88 137.77) (width 0.2) (layer "B.Cu") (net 3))
 (segment (start 44.065 137.825) (end 46.565 137.825) (width 0.2) (layer "B.Cu") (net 3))
 (segment (start 54.73 138.92) (end 55.88 137.77) (width 0.2) (layer "B.Cu") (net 3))
 (segment (start 47.66 138.92) (end 54.73 138.92) (width 0.2) (layer "B.Cu") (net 3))
 (segment (start 33.5 133.77) (end 38.5 133.77) (width 0.2) (layer "F.Cu") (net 27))
 (segment (start 33 134.27) (end 33.5 133.77) (width 0.2) (layer "F.Cu") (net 27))
 (segment (start 33 135.27) (end 33 134.27) (width 0.2) (layer "F.Cu") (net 27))
 (via (at 38.5 133.77) (size 0.6) (drill 0.3) (layers "F.Cu" "B.Cu") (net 27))
 (segment (start 39.865 134.135) (end 39.5 133.77) (width 0.2) (layer "B.Cu") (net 27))
 (segment (start 39.5 133.77) (end 38.5 133.77) (width 0.2) (layer "B.Cu") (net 27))
 (segment (start 49.69 134.135) (end 50.825 135.27) (width 0.2) (layer "B.Cu") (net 27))
 (segment (start 39.865 134.135) (end 49.69 134.135) (width 0.2) (layer "B.Cu") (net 27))
 (segment (start 29.6 134.67) (end 29.6 135.27) (width 0.2) (layer "F.Cu") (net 23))
 (segment (start 31.297057 132.972943) (end 29.6 134.67) (width 0.2) (layer "F.Cu") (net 23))
 (segment (start 31.297057 131.67) (end 31.297057 132.972943) (width 0.2) (layer "F.Cu") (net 23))
 (via (at 31.297057 131.67) (size 0.6) (drill 0.3) (layers "F.Cu" "B.Cu") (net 23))
 (segment (start 31.297057 131.67) (end 31.772057 131.195) (width 0.2) (layer "B.Cu") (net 23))
 (segment (start 48.965 132.77) (end 50.825 132.77) (width 0.2) (layer "B.Cu") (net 23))
 (segment (start 47.39 131.195) (end 48.965 132.77) (width 0.2) (layer "B.Cu") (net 23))
 (segment (start 31.772057 131.195) (end 47.39 131.195) (width 0.2) (layer "B.Cu") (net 23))
 (segment (start 27.9 134.37) (end 28 134.27) (width 0.2) (layer "F.Cu") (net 1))
 (segment (start 27.9 135.27) (end 27.9 134.37) (width 0.2) (layer "F.Cu") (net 1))
 (via (at 28 134.27) (size 0.6) (drill 0.3) (layers "F.Cu" "B.Cu") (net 1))
 (segment (start 31.348529 130.77) (end 30.748529 131.37) (width 0.2) (layer "B.Cu") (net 1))
 (segment (start 30.1 131.37) (end 29.9 131.17) (width 0.2) (layer "B.Cu") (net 1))
 (segment (start 48.425685 130.77) (end 48.925685 130.27) (width 0.2) (layer "B.Cu") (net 1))
 (segment (start 48.925685 130.27) (end 50.785 130.27) (width 0.2) (layer "B.Cu") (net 1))
 (segment (start 29.9 131.17) (end 29.251471 131.17) (width 0.2) (layer "B.Cu") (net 1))
 (segment (start 28 132.421471) (end 28 134.27) (width 0.2) (layer "B.Cu") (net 1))
 (segment (start 30.748529 131.37) (end 30.1 131.37) (width 0.2) (layer "B.Cu") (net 1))
 (segment (start 29.251471 131.17) (end 28 132.421471) (width 0.2) (layer "B.Cu") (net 1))
 (segment (start 31.348529 130.77) (end 48.425685 130.77) (width 0.2) (layer "B.Cu") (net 1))
 (segment (start 27.05 129.97) (end 29.5 127.52) (width 0.2) (layer "F.Cu") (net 17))
 (segment (start 29.5 127.52) (end 29.5 127.27) (width 0.2) (layer "F.Cu") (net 17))
 (segment (start 26.85 129.97) (end 27.05 129.97) (width 0.2) (layer "F.Cu") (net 17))
 (via (at 29.5 127.27) (size 0.6) (drill 0.3) (layers "F.Cu" "B.Cu") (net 17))
 (segment (start 44 123.77) (end 33 123.77) (width 0.2) (layer "B.Cu") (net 17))
 (segment (start 33 123.77) (end 29.5 127.27) (width 0.2) (layer "B.Cu") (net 17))
 (segment (start 27.05 128.27) (end 28.5 126.82) (width 0.2) (layer "F.Cu") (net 15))
 (segment (start 26.85 128.27) (end 27.05 128.27) (width 0.2) (layer "F.Cu") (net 15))
 (segment (start 28.5 126.82) (end 28.5 126.27) (width 0.2) (layer "F.Cu") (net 15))
 (via (at 28.5 126.27) (size 0.6) (drill 0.3) (layers "F.Cu" "B.Cu") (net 15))
 (segment (start 45.35 122.62) (end 32.15 122.62) (width 0.2) (layer "B.Cu") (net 15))
 (segment (start 46.5 123.77) (end 45.35 122.62) (width 0.2) (layer "B.Cu") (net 15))
 (segment (start 32.15 122.62) (end 28.5 126.27) (width 0.2) (layer "B.Cu") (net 15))
 (segment (start 28.875 133.37) (end 26.85 133.37) (width 0.2) (layer "F.Cu") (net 21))
 (segment (start 29.5 132.745) (end 28.875 133.37) (width 0.2) (layer "F.Cu") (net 21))
 (via (at 29.5 132.745) (size 0.6) (drill 0.3) (layers "F.Cu" "B.Cu") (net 21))
 (segment (start 29.5 132.745) (end 44.065 132.745) (width 0.2) (layer "B.Cu") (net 21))
 (segment (start 29.4 131.67) (end 26.85 131.67) (width 0.2) (layer "F.Cu") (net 19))
 (segment (start 29.5 131.77) (end 29.4 131.67) (width 0.2) (layer "F.Cu") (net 19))
 (via (at 29.5 131.77) (size 0.6) (drill 0.3) (layers "F.Cu" "B.Cu") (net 19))
 (segment (start 29.5 131.77) (end 30 132.27) (width 0.2) (layer "B.Cu") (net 19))
 (segment (start 30 132.27) (end 41.5 132.27) (width 0.2) (layer "B.Cu") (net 19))
 (segment (start 41.5 132.27) (end 42.175 131.595) (width 0.2) (layer "B.Cu") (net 19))
 (segment (start 42.175 131.595) (end 45.415 131.595) (width 0.2) (layer "B.Cu") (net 19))
 (segment (start 45.415 131.595) (end 46.565 132.745) (width 0.2) (layer "B.Cu") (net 19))
 (segment (start 28.75 134.57) (end 28.75 135.27) (width 0.2) (layer "F.Cu") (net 9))
 (segment (start 30.5 132.82) (end 28.75 134.57) (width 0.2) (layer "F.Cu") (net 9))
 (segment (start 30.5 130.77) (end 30.5 132.82) (width 0.2) (layer "F.Cu") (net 9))
 (via (at 30.5 130.77) (size 0.6) (drill 0.3) (layers "F.Cu" "B.Cu") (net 9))
 (segment (start 48.26 130.37) (end 48.26 130.31) (width 0.2) (layer "B.Cu") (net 9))
 (segment (start 30.9 130.37) (end 48.26 130.37) (width 0.2) (layer "B.Cu") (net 9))
 (segment (start 48.26 130.31) (end 50.8 127.77) (width 0.2) (layer "B.Cu") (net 9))
 (segment (start 30.5 130.77) (end 30.9 130.37) (width 0.2) (layer "B.Cu") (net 9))
 (segment (start 36.45 130.82) (end 32.95 130.82) (width 0.2) (layer "F.Cu") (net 24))
 (segment (start 32.95 130.82) (end 31.897057 131.872943) (width 0.2) (layer "F.Cu") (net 24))
 (segment (start 37.5 129.77) (end 36.45 130.82) (width 0.2) (layer "F.Cu") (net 24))
 (segment (start 31.897057 131.872943) (end 31.897057 132.938629) (width 0.2) (layer "F.Cu") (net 24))
 (segment (start 30.45 134.385686) (end 30.45 135.27) (width 0.2) (layer "F.Cu") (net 24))
 (segment (start 31.897057 132.938629) (end 30.45 134.385686) (width 0.2) (layer "F.Cu") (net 24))
 (via (at 37.5 129.77) (size 0.6) (drill 0.3) (layers "F.Cu" "B.Cu") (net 24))
 (segment (start 50.8 125.47) (end 50.8 125.27) (width 0.2) (layer "B.Cu") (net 24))
 (segment (start 41.158529 127.46) (end 48.81 127.46) (width 0.2) (layer "B.Cu") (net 24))
 (segment (start 41.158529 127.46) (end 38.848529 129.77) (width 0.2) (layer "B.Cu") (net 24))
 (segment (start 48.81 127.46) (end 50.8 125.47) (width 0.2) (layer "B.Cu") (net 24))
 (segment (start 38.848529 129.77) (end 37.5 129.77) (width 0.2) (layer "B.Cu") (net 24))
 (segment (start 35.6 133.17) (end 33.534314 133.17) (width 0.2) (layer "F.Cu") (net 26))
 (segment (start 39.5 129.27) (end 35.6 133.17) (width 0.2) (layer "F.Cu") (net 26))
 (segment (start 33.534314 133.17) (end 32.15 134.554314) (width 0.2) (layer "F.Cu") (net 26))
 (segment (start 39.5 128.27) (end 39.5 129.27) (width 0.2) (layer "F.Cu") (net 26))
 (segment (start 32.15 134.554314) (end 32.15 135.27) (width 0.2) (layer "F.Cu") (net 26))
 (via (at 39.5 128.27) (size 0.6) (drill 0.3) (layers "F.Cu" "B.Cu") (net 26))
 (segment (start 48.26 125.16) (end 50.65 122.77) (width 0.2) (layer "B.Cu") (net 26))
 (segment (start 42.61 125.16) (end 48.26 125.16) (width 0.2) (layer "B.Cu") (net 26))
 (segment (start 50.65 122.77) (end 50.8 122.77) (width 0.2) (layer "B.Cu") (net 26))
 (segment (start 39.5 128.27) (end 42.61 125.16) (width 0.2) (layer "B.Cu") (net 26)))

